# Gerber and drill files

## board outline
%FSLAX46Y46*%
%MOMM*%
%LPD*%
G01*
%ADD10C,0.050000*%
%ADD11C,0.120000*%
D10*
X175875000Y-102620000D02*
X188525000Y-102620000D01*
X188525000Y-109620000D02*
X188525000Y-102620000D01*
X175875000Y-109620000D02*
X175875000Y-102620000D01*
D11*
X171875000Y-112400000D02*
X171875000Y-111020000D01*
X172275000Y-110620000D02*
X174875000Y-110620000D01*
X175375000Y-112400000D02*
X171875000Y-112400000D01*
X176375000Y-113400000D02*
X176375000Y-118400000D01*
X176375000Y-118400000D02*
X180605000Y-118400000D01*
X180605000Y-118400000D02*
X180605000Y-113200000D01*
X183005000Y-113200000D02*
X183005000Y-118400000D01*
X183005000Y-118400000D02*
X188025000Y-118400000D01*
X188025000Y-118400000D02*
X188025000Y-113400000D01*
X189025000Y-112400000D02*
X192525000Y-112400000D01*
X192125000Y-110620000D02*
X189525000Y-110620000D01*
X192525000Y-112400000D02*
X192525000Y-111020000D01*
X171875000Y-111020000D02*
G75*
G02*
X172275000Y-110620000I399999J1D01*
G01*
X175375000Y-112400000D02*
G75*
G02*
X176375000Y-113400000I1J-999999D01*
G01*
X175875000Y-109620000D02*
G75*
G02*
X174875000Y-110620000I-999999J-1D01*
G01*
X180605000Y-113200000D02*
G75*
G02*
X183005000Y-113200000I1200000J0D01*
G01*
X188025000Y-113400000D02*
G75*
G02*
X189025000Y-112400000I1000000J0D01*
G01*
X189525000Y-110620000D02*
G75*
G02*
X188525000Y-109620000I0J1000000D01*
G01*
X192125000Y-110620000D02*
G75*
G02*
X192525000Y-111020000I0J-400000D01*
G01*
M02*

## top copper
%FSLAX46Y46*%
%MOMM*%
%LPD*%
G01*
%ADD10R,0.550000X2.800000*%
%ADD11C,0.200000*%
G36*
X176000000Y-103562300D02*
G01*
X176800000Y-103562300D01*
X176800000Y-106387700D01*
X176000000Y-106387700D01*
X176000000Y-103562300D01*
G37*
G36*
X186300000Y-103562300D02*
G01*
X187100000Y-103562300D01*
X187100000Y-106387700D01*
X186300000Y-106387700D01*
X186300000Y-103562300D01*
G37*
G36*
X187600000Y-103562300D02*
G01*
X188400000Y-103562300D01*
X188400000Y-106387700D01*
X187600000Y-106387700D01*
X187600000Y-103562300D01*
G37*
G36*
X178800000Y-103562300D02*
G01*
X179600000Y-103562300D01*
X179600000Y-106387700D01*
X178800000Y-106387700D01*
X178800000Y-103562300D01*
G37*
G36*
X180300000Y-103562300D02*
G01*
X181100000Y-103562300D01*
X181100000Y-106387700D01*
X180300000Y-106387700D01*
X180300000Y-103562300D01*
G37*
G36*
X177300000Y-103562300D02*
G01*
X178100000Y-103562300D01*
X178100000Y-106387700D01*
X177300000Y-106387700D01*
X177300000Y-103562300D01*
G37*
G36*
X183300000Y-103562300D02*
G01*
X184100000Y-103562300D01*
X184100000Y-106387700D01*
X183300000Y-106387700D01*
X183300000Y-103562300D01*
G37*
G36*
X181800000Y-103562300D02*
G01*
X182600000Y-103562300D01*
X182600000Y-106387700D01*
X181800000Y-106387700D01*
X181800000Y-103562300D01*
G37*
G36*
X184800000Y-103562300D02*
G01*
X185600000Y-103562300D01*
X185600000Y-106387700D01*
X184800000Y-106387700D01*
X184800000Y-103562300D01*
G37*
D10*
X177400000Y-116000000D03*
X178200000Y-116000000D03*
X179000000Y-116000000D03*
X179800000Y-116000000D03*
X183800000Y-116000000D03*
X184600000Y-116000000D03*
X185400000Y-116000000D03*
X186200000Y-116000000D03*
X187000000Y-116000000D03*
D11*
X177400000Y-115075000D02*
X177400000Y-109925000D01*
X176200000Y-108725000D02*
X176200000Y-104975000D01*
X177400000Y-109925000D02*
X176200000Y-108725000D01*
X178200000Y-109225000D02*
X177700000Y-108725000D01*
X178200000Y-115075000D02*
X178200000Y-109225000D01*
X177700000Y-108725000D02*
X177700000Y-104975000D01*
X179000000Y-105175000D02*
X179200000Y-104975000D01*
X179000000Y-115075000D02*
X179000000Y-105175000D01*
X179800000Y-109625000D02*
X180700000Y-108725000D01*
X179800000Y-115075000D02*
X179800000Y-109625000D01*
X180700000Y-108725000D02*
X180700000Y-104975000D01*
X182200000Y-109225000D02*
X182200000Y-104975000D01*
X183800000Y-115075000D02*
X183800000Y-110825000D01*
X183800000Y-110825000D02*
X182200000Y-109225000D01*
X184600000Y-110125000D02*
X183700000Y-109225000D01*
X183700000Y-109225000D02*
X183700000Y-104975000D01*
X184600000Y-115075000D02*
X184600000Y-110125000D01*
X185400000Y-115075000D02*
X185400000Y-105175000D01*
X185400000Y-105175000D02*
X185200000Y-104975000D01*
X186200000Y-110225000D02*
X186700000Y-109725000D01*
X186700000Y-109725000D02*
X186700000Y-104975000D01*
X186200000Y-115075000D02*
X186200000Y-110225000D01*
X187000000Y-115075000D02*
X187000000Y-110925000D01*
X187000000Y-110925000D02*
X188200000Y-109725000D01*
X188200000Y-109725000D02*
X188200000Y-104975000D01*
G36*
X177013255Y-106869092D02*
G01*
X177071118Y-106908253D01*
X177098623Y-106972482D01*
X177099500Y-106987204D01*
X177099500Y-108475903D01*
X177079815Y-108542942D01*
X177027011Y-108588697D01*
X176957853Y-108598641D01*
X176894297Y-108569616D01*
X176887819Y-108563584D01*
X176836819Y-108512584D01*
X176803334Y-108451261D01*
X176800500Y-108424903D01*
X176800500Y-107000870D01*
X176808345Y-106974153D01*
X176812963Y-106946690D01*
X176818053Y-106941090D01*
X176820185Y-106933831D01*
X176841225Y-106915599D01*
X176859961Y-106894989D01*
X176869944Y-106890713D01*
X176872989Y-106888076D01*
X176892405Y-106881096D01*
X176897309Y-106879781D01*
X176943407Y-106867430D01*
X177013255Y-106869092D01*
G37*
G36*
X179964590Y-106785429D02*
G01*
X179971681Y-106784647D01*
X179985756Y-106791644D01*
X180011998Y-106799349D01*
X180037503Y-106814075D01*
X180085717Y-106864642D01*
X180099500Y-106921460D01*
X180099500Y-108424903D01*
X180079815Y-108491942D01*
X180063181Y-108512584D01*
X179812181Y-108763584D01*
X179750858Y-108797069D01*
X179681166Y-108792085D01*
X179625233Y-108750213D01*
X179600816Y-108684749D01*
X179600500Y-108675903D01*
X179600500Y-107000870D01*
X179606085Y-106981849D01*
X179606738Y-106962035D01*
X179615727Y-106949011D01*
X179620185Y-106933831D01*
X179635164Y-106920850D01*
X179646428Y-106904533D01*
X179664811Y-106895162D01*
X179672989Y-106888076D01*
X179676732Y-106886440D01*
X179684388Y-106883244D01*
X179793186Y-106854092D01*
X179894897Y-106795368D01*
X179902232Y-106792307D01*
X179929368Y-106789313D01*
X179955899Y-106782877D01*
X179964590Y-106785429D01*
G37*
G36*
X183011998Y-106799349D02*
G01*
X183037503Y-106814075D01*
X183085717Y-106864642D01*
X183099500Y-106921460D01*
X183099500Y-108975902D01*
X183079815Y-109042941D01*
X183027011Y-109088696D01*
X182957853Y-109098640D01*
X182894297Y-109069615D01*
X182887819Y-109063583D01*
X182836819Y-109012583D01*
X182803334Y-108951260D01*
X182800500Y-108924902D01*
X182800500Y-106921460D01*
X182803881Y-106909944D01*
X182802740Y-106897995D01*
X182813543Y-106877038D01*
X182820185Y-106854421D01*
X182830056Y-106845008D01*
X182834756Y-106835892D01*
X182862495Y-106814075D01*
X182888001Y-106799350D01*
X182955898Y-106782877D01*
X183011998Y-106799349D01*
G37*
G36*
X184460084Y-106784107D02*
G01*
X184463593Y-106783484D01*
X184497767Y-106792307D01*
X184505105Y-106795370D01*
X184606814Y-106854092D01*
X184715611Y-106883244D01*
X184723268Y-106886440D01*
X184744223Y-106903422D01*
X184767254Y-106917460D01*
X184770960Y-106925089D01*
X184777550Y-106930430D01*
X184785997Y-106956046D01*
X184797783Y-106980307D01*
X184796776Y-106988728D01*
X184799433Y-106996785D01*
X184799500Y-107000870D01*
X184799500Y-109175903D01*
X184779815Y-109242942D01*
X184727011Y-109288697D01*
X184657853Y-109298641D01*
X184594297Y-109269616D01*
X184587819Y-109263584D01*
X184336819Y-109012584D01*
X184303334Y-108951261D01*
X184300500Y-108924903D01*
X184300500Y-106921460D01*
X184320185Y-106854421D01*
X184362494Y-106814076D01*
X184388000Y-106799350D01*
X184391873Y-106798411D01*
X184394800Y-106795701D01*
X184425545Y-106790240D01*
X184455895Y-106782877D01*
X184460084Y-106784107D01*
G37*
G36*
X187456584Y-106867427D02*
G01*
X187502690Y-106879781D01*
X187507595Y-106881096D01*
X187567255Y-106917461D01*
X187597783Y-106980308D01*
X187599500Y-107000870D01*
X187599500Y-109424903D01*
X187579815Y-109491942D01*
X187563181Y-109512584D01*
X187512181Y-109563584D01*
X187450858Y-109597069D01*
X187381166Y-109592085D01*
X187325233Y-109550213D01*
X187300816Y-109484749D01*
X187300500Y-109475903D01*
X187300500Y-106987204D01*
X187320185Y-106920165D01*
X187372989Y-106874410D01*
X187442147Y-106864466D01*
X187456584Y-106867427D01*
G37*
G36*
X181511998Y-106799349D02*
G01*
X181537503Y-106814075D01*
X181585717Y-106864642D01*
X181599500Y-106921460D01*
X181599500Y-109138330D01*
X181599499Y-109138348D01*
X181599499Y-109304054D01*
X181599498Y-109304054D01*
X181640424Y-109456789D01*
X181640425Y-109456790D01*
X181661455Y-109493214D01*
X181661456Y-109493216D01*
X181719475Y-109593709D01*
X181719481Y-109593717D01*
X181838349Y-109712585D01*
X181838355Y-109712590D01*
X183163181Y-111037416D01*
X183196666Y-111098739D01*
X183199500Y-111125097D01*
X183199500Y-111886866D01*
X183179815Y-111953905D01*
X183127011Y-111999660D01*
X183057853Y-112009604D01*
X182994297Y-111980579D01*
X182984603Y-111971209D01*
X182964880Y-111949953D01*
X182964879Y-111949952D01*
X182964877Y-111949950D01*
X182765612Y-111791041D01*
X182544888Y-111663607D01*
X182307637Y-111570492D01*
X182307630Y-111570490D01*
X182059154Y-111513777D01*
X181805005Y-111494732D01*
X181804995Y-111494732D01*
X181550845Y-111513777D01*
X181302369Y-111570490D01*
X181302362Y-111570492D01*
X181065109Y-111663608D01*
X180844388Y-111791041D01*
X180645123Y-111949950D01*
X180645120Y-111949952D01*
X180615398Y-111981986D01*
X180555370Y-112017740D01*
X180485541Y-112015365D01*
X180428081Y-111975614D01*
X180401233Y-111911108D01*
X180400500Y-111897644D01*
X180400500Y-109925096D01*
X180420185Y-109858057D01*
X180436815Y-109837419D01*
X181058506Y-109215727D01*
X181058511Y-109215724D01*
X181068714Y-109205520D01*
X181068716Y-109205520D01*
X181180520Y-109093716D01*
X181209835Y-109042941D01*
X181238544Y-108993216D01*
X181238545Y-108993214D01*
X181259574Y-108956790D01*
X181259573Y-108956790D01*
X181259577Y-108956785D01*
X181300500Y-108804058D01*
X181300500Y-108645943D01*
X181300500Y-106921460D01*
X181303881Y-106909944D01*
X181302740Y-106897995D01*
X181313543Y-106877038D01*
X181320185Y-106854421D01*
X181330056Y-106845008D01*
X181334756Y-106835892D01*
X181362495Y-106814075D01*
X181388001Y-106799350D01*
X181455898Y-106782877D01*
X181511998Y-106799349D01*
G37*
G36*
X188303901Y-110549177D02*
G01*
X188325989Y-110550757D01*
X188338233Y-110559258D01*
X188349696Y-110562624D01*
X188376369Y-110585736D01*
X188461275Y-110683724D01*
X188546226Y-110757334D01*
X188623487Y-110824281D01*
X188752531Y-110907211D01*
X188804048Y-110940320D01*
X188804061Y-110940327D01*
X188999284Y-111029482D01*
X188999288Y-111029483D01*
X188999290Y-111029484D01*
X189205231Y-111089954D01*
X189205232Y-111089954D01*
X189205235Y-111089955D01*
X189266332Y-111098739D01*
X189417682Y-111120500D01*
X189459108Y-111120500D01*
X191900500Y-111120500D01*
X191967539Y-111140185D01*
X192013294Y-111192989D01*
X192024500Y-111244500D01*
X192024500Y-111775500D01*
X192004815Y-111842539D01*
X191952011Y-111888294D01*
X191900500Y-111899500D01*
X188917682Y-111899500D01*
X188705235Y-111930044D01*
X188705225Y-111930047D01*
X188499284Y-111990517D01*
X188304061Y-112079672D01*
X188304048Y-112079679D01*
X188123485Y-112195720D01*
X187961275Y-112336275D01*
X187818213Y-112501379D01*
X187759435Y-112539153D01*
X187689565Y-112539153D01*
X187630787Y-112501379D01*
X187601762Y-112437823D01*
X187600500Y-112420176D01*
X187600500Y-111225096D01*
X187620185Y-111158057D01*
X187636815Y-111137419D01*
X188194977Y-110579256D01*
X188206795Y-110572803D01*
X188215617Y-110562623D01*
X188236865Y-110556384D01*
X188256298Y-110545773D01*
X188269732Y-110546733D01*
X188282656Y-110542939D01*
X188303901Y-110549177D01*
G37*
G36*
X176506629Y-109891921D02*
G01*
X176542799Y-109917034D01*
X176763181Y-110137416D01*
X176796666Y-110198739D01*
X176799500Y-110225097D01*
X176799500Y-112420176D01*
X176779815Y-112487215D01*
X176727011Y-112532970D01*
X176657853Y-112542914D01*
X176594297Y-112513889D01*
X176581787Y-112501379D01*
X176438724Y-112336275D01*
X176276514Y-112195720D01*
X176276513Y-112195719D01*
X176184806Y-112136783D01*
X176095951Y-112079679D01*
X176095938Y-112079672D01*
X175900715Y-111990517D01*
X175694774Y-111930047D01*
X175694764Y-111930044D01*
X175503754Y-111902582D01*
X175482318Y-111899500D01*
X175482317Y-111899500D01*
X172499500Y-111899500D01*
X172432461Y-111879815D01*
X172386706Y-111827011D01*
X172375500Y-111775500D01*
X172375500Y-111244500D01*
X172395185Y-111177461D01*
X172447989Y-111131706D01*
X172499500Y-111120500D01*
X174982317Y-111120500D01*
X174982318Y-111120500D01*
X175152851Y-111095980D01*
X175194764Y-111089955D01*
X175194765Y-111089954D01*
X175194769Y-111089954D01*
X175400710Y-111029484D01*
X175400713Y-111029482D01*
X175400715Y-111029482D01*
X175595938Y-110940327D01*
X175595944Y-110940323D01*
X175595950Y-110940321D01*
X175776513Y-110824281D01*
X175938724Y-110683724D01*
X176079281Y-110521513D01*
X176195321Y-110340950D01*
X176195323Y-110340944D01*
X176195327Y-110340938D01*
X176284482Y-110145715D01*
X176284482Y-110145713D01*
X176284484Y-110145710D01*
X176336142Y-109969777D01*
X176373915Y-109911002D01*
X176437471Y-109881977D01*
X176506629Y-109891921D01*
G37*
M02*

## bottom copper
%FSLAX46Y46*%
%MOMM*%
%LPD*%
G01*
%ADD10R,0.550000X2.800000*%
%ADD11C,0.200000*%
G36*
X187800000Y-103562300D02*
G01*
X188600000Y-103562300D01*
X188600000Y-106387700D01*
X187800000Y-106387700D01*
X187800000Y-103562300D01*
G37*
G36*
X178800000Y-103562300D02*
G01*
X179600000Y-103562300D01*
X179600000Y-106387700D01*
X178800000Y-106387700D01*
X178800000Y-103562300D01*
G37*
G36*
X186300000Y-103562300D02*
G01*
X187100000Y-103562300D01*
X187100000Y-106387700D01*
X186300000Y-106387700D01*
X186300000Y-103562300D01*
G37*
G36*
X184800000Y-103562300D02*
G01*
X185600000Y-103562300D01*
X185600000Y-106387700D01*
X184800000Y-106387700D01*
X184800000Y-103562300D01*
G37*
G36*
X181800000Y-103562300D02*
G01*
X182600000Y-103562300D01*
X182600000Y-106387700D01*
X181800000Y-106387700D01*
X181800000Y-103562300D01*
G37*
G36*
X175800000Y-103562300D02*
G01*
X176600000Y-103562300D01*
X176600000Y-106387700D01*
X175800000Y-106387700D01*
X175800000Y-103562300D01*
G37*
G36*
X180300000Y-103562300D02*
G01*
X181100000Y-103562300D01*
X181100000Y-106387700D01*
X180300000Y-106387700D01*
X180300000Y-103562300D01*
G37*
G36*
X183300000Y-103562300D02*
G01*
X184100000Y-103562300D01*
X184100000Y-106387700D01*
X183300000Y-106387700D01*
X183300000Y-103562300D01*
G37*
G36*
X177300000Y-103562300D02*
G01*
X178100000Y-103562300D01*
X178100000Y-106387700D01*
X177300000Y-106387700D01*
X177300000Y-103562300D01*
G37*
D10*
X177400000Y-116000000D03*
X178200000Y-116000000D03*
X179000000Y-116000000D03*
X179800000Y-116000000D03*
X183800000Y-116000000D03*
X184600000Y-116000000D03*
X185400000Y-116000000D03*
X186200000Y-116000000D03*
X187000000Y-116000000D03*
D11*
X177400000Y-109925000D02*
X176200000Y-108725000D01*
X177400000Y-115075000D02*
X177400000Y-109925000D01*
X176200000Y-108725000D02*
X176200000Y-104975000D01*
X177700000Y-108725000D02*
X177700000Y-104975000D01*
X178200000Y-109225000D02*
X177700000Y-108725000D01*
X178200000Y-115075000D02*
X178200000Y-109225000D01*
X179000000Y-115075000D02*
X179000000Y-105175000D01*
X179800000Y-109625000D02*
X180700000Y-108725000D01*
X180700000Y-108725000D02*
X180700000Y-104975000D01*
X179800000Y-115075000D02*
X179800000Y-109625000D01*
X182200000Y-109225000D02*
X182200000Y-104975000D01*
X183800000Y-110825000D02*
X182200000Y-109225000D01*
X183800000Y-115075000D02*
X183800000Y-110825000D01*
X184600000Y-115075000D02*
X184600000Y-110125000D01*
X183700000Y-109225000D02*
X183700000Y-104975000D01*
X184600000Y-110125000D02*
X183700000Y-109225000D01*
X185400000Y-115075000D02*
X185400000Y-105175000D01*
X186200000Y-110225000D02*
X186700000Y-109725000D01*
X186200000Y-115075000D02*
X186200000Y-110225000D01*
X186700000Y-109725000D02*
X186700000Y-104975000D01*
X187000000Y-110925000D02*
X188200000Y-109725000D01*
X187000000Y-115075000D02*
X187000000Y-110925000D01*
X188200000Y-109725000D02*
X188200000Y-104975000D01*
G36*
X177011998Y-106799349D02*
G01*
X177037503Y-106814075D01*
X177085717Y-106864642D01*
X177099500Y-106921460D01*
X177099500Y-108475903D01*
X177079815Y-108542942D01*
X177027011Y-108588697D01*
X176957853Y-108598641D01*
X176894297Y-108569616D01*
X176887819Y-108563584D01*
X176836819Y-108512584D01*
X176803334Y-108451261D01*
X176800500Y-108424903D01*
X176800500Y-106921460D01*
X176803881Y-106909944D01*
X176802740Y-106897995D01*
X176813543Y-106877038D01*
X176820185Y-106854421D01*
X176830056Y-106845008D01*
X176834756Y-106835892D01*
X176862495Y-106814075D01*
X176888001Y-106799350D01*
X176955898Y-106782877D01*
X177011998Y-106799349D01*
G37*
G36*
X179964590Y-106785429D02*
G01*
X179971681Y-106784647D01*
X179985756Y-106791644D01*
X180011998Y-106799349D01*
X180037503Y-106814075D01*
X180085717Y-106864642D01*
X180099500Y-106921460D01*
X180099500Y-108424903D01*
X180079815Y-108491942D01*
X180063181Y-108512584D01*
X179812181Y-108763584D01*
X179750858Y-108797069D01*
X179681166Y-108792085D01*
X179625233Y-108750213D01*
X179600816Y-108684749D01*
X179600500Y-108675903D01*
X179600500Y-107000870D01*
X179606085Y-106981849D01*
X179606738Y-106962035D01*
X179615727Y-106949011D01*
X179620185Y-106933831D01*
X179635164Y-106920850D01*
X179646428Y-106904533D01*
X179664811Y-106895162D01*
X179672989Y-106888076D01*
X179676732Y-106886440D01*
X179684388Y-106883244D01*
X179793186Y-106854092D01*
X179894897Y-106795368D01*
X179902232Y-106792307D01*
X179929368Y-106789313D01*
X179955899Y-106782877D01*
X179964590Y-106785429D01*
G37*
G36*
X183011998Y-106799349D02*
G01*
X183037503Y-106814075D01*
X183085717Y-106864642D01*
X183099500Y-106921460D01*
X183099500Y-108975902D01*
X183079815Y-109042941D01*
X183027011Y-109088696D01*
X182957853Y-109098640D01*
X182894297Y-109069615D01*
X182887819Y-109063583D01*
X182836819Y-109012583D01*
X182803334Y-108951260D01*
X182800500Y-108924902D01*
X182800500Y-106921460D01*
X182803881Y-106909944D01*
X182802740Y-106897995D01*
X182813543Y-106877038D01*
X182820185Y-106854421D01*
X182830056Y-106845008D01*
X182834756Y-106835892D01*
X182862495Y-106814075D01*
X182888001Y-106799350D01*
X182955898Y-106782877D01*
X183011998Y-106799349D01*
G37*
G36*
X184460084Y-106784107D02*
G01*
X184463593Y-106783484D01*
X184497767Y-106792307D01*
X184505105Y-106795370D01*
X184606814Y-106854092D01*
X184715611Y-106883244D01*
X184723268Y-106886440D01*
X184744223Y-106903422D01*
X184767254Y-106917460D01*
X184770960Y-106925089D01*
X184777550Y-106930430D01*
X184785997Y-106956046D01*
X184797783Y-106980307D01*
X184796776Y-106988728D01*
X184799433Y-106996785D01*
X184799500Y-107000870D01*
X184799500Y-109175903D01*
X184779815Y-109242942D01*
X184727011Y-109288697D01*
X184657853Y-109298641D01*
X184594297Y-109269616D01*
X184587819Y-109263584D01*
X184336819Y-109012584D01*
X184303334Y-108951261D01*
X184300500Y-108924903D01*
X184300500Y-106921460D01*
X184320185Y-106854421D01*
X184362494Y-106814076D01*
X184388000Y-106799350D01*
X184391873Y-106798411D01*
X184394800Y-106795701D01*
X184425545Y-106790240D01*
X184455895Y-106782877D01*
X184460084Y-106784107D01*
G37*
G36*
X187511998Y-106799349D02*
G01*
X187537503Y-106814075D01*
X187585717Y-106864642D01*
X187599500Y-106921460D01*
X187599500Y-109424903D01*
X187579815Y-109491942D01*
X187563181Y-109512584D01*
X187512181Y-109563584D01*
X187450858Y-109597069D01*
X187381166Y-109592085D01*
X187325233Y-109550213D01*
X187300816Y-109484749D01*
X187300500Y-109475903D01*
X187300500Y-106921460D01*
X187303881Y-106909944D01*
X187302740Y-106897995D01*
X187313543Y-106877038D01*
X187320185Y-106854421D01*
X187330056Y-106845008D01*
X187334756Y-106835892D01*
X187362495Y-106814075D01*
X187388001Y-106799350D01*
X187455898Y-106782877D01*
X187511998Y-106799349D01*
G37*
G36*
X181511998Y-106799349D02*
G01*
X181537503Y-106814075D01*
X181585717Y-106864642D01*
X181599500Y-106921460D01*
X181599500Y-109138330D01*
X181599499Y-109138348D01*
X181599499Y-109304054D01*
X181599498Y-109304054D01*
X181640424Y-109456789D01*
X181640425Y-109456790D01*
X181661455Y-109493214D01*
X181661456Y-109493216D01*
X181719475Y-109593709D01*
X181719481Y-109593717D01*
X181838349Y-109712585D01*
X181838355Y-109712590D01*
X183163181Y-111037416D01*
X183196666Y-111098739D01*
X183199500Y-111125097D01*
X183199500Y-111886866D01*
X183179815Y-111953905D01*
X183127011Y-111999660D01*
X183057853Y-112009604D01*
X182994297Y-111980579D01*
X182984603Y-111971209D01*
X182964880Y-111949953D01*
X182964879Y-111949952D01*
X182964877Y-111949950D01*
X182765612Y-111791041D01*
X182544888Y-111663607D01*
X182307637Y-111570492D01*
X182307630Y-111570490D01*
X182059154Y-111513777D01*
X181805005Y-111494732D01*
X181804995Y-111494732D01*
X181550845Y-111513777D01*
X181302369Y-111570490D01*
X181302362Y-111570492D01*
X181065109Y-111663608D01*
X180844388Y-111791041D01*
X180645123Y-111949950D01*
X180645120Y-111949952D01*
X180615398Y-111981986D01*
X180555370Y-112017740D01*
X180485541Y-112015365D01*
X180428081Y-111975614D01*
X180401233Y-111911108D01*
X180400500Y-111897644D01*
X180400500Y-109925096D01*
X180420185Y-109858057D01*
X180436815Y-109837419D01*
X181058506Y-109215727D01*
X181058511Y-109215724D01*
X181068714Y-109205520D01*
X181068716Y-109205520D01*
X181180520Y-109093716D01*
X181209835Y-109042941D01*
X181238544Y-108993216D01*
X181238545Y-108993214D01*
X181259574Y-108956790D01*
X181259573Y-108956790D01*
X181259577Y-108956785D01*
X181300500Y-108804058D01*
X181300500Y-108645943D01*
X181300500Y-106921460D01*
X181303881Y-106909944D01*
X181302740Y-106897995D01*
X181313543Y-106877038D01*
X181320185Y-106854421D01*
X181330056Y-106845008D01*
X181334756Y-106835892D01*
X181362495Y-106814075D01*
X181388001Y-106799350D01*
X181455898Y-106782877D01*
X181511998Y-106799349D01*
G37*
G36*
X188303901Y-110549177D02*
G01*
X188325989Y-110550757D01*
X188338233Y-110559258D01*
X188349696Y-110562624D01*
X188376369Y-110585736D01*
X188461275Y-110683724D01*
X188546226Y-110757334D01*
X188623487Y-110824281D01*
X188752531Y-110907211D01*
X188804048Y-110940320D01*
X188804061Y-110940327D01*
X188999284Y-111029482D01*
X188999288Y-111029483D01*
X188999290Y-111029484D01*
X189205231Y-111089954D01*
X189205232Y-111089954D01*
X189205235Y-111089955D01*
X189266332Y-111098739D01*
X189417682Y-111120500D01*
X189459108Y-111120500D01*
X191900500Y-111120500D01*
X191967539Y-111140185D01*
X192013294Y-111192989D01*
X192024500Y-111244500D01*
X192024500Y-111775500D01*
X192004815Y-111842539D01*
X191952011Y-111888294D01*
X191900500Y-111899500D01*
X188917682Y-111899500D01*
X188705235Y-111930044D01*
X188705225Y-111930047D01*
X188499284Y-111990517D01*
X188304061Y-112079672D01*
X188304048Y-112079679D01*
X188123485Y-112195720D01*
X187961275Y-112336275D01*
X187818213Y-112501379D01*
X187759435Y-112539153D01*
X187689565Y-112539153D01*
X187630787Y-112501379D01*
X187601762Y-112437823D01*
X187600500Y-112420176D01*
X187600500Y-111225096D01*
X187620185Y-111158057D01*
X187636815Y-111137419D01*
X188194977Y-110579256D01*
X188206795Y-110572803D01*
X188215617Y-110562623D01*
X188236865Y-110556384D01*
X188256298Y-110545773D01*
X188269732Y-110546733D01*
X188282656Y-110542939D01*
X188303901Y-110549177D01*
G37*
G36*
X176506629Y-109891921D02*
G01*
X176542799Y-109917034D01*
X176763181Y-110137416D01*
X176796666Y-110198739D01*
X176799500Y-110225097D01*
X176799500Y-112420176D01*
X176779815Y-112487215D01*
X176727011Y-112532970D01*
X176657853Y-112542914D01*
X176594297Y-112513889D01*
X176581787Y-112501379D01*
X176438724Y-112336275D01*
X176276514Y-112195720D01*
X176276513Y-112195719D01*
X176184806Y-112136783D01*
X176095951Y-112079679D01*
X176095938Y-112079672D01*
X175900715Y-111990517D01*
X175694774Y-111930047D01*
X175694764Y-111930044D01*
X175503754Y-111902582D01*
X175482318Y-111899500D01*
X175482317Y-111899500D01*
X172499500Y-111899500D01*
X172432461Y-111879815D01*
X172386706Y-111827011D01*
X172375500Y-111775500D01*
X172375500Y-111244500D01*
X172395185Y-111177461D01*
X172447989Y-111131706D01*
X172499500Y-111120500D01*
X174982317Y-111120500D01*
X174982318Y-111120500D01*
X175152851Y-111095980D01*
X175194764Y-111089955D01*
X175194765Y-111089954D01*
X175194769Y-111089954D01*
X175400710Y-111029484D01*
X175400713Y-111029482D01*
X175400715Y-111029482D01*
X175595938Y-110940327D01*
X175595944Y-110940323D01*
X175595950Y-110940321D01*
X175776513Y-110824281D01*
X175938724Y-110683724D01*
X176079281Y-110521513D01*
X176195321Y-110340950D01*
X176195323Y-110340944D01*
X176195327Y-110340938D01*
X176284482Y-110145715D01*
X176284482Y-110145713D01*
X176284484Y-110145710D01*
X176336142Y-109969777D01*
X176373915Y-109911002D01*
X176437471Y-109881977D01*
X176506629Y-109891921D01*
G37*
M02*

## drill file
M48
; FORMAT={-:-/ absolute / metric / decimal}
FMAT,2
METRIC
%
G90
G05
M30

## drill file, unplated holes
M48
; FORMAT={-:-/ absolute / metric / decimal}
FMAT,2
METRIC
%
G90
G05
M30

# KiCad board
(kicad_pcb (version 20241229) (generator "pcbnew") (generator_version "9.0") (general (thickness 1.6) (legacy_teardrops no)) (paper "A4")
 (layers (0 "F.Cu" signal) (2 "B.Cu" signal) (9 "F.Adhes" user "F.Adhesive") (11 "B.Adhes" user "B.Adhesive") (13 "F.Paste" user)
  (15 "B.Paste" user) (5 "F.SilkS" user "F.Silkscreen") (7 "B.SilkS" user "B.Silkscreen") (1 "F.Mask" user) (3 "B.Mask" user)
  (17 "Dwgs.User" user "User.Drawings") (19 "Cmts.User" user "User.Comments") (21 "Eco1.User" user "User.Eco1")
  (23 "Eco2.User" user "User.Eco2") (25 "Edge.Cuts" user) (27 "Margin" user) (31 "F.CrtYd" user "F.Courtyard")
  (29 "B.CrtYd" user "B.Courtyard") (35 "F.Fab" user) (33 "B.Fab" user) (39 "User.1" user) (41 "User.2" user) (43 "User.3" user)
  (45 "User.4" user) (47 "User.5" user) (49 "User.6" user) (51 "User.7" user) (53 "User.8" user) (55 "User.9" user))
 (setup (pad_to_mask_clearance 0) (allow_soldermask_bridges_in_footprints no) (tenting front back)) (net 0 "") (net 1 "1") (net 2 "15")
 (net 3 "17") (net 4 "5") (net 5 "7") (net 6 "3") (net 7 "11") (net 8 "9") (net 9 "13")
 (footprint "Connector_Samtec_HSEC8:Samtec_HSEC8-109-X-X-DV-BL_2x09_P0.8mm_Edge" (layer "F.Cu") (at 182.2 118.4)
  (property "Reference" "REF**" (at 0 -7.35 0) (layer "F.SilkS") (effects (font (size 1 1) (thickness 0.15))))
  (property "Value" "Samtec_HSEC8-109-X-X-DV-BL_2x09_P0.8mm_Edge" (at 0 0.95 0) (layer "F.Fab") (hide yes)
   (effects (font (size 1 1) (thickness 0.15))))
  (fp_line (start -10.325 -6) (end -10.325 -7.38) (stroke (width 0.12) (type solid)) (layer "Edge.Cuts"))
  (fp_line (start -9.925 -7.78) (end -7.325 -7.78) (stroke (width 0.12) (type solid)) (layer "Edge.Cuts"))
  (fp_line (start -6.825 -6) (end -10.325 -6) (stroke (width 0.12) (type solid)) (layer "Edge.Cuts"))
  (fp_line (start -5.825 -5) (end -5.825 0) (stroke (width 0.12) (type solid)) (layer "Edge.Cuts"))
  (fp_line (start -5.825 0) (end -1.595 0) (stroke (width 0.12) (type solid)) (layer "Edge.Cuts"))
  (fp_line (start -1.595 0) (end -1.595 -5.2) (stroke (width 0.12) (type solid)) (layer "Edge.Cuts"))
  (fp_line (start 0.805 -5.2) (end 0.805 0) (stroke (width 0.12) (type solid)) (layer "Edge.Cuts"))
  (fp_line (start 0.805 0) (end 5.825 0) (stroke (width 0.12) (type solid)) (layer "Edge.Cuts"))
  (fp_line (start 5.825 0) (end 5.825 -5) (stroke (width 0.12) (type solid)) (layer "Edge.Cuts"))
  (fp_line (start 6.825 -6) (end 10.325 -6) (stroke (width 0.12) (type solid)) (layer "Edge.Cuts"))
  (fp_line (start 9.925 -7.78) (end 7.325 -7.78) (stroke (width 0.12) (type solid)) (layer "Edge.Cuts"))
  (fp_line (start 10.325 -6) (end 10.325 -7.38) (stroke (width 0.12) (type solid)) (layer "Edge.Cuts"))
  (fp_arc (start -10.325 -7.38) (mid -10.207843 -7.662843) (end -9.925 -7.78) (stroke (width 0.12) (type solid)) (layer "Edge.Cuts"))
  (fp_arc (start -6.825 -6) (mid -6.117893 -5.707107) (end -5.825 -5) (stroke (width 0.12) (type solid)) (layer "Edge.Cuts"))
  (fp_arc (start -6.325 -8.78) (mid -6.617893 -8.072893) (end -7.325 -7.78) (stroke (width 0.12) (type solid)) (layer "Edge.Cuts"))
  (fp_arc (start -1.595 -5.2) (mid -0.395 -6.4) (end 0.805 -5.2) (stroke (width 0.12) (type solid)) (layer "Edge.Cuts"))
  (fp_arc (start 5.825 -5) (mid 6.117893 -5.707107) (end 6.825 -6) (stroke (width 0.12) (type solid)) (layer "Edge.Cuts"))
  (fp_arc (start 7.325 -7.78) (mid 6.617893 -8.072893) (end 6.325 -8.78) (stroke (width 0.12) (type solid)) (layer "Edge.Cuts"))
  (fp_arc (start 9.925 -7.78) (mid 10.207843 -7.662843) (end 10.325 -7.38) (stroke (width 0.12) (type solid)) (layer "Edge.Cuts"))
  (pad "1" connect rect (at -4.8 -2.4) (size 0.55 2.8) (layers "F.Cu" "F.Mask"))
  (pad "2" connect rect (at -4.8 -2.4) (size 0.55 2.8) (layers "B.Cu" "B.Mask"))
  (pad "3" connect rect (at -4 -2.4) (size 0.55 2.8) (layers "F.Cu" "F.Mask"))
  (pad "4" connect rect (at -4 -2.4) (size 0.55 2.8) (layers "B.Cu" "B.Mask"))
  (pad "5" connect rect (at -3.2 -2.4) (size 0.55 2.8) (layers "F.Cu" "F.Mask"))
  (pad "6" connect rect (at -3.2 -2.4) (size 0.55 2.8) (layers "B.Cu" "B.Mask"))
  (pad "7" connect rect (at -2.4 -2.4) (size 0.55 2.8) (layers "F.Cu" "F.Mask"))
  (pad "8" connect rect (at -2.4 -2.4) (size 0.55 2.8) (layers "B.Cu" "B.Mask"))
  (pad "9" connect rect (at 1.6 -2.4) (size 0.55 2.8) (layers "F.Cu" "F.Mask"))
  (pad "10" connect rect (at 1.6 -2.4) (size 0.55 2.8) (layers "B.Cu" "B.Mask"))
  (pad "11" connect rect (at 2.4 -2.4) (size 0.55 2.8) (layers "F.Cu" "F.Mask"))
  (pad "12" connect rect (at 2.4 -2.4) (size 0.55 2.8) (layers "B.Cu" "B.Mask"))
  (pad "13" connect rect (at 3.2 -2.4) (size 0.55 2.8) (layers "F.Cu" "F.Mask"))
  (pad "14" connect rect (at 3.2 -2.4) (size 0.55 2.8) (layers "B.Cu" "B.Mask"))
  (pad "15" connect rect (at 4 -2.4) (size 0.55 2.8) (layers "F.Cu" "F.Mask"))
  (pad "16" connect rect (at 4 -2.4) (size 0.55 2.8) (layers "B.Cu" "B.Mask"))
  (pad "17" connect rect (at 4.8 -2.4) (size 0.55 2.8) (layers "F.Cu" "F.Mask"))
  (pad "18" connect rect (at 4.8 -2.4) (size 0.55 2.8) (layers "B.Cu" "B.Mask")))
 (gr_rect (start 176 103.5623) (end 176.8 106.3877) (stroke (width 0) (type solid)) (fill yes) (layer "F.Cu") (net 1))
 (gr_rect (start 186.3 103.5623) (end 187.1 106.3877) (stroke (width 0) (type solid)) (fill yes) (layer "F.Cu") (net 2))
 (gr_rect (start 187.6 103.5623) (end 188.4 106.3877) (stroke (width 0) (type solid)) (fill yes) (layer "F.Cu") (net 3))
 (gr_rect (start 178.8 103.5623) (end 179.6 106.3877) (stroke (width 0) (type solid)) (fill yes) (layer "F.Cu") (net 4))
 (gr_rect (start 180.3 103.5623) (end 181.1 106.3877) (stroke (width 0) (type solid)) (fill yes) (layer "F.Cu") (net 5))
 (gr_rect (start 177.3 103.5623) (end 178.1 106.3877) (stroke (width 0) (type solid)) (fill yes) (layer "F.Cu") (net 6))
 (gr_rect (start 183.3 103.5623) (end 184.1 106.3877) (stroke (width 0) (type solid)) (fill yes) (layer "F.Cu") (net 7))
 (gr_rect (start 181.8 103.5623) (end 182.6 106.3877) (stroke (width 0) (type solid)) (fill yes) (layer "F.Cu") (net 8))
 (gr_rect (start 184.8 103.5623) (end 185.6 106.3877) (stroke (width 0) (type solid)) (fill yes) (layer "F.Cu") (net 9))
 (gr_rect (start 187.8 103.5623) (end 188.6 106.3877) (stroke (width 0) (type solid)) (fill yes) (layer "B.Cu") (net 3))
 (gr_rect (start 178.8 103.5623) (end 179.6 106.3877) (stroke (width 0) (type solid)) (fill yes) (layer "B.Cu") (net 4))
 (gr_rect (start 186.3 103.5623) (end 187.1 106.3877) (stroke (width 0) (type solid)) (fill yes) (layer "B.Cu") (net 2))
 (gr_rect (start 184.8 103.5623) (end 185.6 106.3877) (stroke (width 0) (type solid)) (fill yes) (layer "B.Cu") (net 9))
 (gr_rect (start 181.8 103.5623) (end 182.6 106.3877) (stroke (width 0) (type solid)) (fill yes) (layer "B.Cu") (net 8))
 (gr_rect (start 175.8 103.5623) (end 176.6 106.3877) (stroke (width 0) (type solid)) (fill yes) (layer "B.Cu") (net 1))
 (gr_rect (start 180.3 103.5623) (end 181.1 106.3877) (stroke (width 0) (type solid)) (fill yes) (layer "B.Cu") (net 5))
 (gr_rect (start 183.3 103.5623) (end 184.1 106.3877) (stroke (width 0) (type solid)) (fill yes) (layer "B.Cu") (net 7))
 (gr_rect (start 177.3 103.5623) (end 178.1 106.3877) (stroke (width 0) (type solid)) (fill yes) (layer "B.Cu") (net 6))
 (gr_line (start 175.875 109.62) (end 175.875 102.62) (stroke (width 0.05) (type solid)) (layer "Edge.Cuts"))
 (gr_line (start 175.875 102.62) (end 188.525 102.62) (stroke (width 0.05) (type default)) (layer "Edge.Cuts"))
 (gr_line (start 188.525 109.62) (end 188.525 102.62) (stroke (width 0.05) (type solid)) (layer "Edge.Cuts"))
 (segment (start 177.4 115.075) (end 177.4 109.925) (width 0.2) (layer "F.Cu") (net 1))
 (segment (start 176.2 108.725) (end 176.2 104.975) (width 0.2) (layer "F.Cu") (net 1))
 (segment (start 177.4 109.925) (end 176.2 108.725) (width 0.2) (layer "F.Cu") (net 1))
 (segment (start 177.4 109.925) (end 176.2 108.725) (width 0.2) (layer "B.Cu") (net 1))
 (segment (start 177.4 115.075) (end 177.4 109.925) (width 0.2) (layer "B.Cu") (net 1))
 (segment (start 176.2 108.725) (end 176.2 104.975) (width 0.2) (layer "B.Cu") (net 1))
 (segment (start 178.2 109.225) (end 177.7 108.725) (width 0.2) (layer "F.Cu") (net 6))
 (segment (start 178.2 115.075) (end 178.2 109.225) (width 0.2) (layer "F.Cu") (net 6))
 (segment (start 177.7 108.725) (end 177.7 104.975) (width 0.2) (layer "F.Cu") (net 6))
 (segment (start 177.7 108.725) (end 177.7 104.975) (width 0.2) (layer "B.Cu") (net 6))
 (segment (start 178.2 109.225) (end 177.7 108.725) (width 0.2) (layer "B.Cu") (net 6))
 (segment (start 178.2 115.075) (end 178.2 109.225) (width 0.2) (layer "B.Cu") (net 6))
 (segment (start 179 105.175) (end 179.2 104.975) (width 0.2) (layer "F.Cu") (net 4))
 (segment (start 179 115.075) (end 179 105.175) (width 0.2) (layer "F.Cu") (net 4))
 (segment (start 179 115.075) (end 179 105.175) (width 0.2) (layer "B.Cu") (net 4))
 (segment (start 179.8 109.625) (end 180.7 108.725) (width 0.2) (layer "F.Cu") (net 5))
 (segment (start 179.8 115.075) (end 179.8 109.625) (width 0.2) (layer "F.Cu") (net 5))
 (segment (start 180.7 108.725) (end 180.7 104.975) (width 0.2) (layer "F.Cu") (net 5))
 (segment (start 179.8 109.625) (end 180.7 108.725) (width 0.2) (layer "B.Cu") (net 5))
 (segment (start 180.7 108.725) (end 180.7 104.975) (width 0.2) (layer "B.Cu") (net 5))
 (segment (start 179.8 115.075) (end 179.8 109.625) (width 0.2) (layer "B.Cu") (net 5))
 (segment (start 182.2 109.225) (end 182.2 104.975) (width 0.2) (layer "F.Cu") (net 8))
 (segment (start 183.8 115.075) (end 183.8 110.825) (width 0.2) (layer "F.Cu") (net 8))
 (segment (start 183.8 110.825) (end 182.2 109.225) (width 0.2) (layer "F.Cu") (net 8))
 (segment (start 182.2 109.225) (end 182.2 104.975) (width 0.2) (layer "B.Cu") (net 8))
 (segment (start 183.8 110.825) (end 182.2 109.225) (width 0.2) (layer "B.Cu") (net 8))
 (segment (start 183.8 115.075) (end 183.8 110.825) (width 0.2) (layer "B.Cu") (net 8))
 (segment (start 184.6 110.125) (end 183.7 109.225) (width 0.2) (layer "F.Cu") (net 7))
 (segment (start 183.7 109.225) (end 183.7 104.975) (width 0.2) (layer "F.Cu") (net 7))
 (segment (start 184.6 115.075) (end 184.6 110.125) (width 0.2) (layer "F.Cu") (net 7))
 (segment (start 184.6 115.075) (end 184.6 110.125) (width 0.2) (layer "B.Cu") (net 7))
 (segment (start 183.7 109.225) (end 183.7 104.975) (width 0.2) (layer "B.Cu") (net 7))
 (segment (start 184.6 110.125) (end 183.7 109.225) (width 0.2) (layer "B.Cu") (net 7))
 (segment (start 185.4 115.075) (end 185.4 105.175) (width 0.2) (layer "F.Cu") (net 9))
 (segment (start 185.4 105.175) (end 185.2 104.975) (width 0.2) (layer "F.Cu") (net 9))
 (segment (start 185.4 115.075) (end 185.4 105.175) (width 0.2) (layer "B.Cu") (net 9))
 (segment (start 186.2 110.225) (end 186.7 109.725) (width 0.2) (layer "F.Cu") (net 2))
 (segment (start 186.7 109.725) (end 186.7 104.975) (width 0.2) (layer "F.Cu") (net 2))
 (segment (start 186.2 115.075) (end 186.2 110.225) (width 0.2) (layer "F.Cu") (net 2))
 (segment (start 186.2 110.225) (end 186.7 109.725) (width 0.2) (layer "B.Cu") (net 2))
 (segment (start 186.2 115.075) (end 186.2 110.225) (width 0.2) (layer "B.Cu") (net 2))
 (segment (start 186.7 109.725) (end 186.7 104.975) (width 0.2) (layer "B.Cu") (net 2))
 (segment (start 187 115.075) (end 187 110.925) (width 0.2) (layer "F.Cu") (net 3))
 (segment (start 187 110.925) (end 188.2 109.725) (width 0.2) (layer "F.Cu") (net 3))
 (segment (start 188.2 109.725) (end 188.2 104.975) (width 0.2) (layer "F.Cu") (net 3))
 (segment (start 187 110.925) (end 188.2 109.725) (width 0.2) (layer "B.Cu") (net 3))
 (segment (start 187 115.075) (end 187 110.925) (width 0.2) (layer "B.Cu") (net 3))
 (segment (start 188.2 109.725) (end 188.2 104.975) (width 0.2) (layer "B.Cu") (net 3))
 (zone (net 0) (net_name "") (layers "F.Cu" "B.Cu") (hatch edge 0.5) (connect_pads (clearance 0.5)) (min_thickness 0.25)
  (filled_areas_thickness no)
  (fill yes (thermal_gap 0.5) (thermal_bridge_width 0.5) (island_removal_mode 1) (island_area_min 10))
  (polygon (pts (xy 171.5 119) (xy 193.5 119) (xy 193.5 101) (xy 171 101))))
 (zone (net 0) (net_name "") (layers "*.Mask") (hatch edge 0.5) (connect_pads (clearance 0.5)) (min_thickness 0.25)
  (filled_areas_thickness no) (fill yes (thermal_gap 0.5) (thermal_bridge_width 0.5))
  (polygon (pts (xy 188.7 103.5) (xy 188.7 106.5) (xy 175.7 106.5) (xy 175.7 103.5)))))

